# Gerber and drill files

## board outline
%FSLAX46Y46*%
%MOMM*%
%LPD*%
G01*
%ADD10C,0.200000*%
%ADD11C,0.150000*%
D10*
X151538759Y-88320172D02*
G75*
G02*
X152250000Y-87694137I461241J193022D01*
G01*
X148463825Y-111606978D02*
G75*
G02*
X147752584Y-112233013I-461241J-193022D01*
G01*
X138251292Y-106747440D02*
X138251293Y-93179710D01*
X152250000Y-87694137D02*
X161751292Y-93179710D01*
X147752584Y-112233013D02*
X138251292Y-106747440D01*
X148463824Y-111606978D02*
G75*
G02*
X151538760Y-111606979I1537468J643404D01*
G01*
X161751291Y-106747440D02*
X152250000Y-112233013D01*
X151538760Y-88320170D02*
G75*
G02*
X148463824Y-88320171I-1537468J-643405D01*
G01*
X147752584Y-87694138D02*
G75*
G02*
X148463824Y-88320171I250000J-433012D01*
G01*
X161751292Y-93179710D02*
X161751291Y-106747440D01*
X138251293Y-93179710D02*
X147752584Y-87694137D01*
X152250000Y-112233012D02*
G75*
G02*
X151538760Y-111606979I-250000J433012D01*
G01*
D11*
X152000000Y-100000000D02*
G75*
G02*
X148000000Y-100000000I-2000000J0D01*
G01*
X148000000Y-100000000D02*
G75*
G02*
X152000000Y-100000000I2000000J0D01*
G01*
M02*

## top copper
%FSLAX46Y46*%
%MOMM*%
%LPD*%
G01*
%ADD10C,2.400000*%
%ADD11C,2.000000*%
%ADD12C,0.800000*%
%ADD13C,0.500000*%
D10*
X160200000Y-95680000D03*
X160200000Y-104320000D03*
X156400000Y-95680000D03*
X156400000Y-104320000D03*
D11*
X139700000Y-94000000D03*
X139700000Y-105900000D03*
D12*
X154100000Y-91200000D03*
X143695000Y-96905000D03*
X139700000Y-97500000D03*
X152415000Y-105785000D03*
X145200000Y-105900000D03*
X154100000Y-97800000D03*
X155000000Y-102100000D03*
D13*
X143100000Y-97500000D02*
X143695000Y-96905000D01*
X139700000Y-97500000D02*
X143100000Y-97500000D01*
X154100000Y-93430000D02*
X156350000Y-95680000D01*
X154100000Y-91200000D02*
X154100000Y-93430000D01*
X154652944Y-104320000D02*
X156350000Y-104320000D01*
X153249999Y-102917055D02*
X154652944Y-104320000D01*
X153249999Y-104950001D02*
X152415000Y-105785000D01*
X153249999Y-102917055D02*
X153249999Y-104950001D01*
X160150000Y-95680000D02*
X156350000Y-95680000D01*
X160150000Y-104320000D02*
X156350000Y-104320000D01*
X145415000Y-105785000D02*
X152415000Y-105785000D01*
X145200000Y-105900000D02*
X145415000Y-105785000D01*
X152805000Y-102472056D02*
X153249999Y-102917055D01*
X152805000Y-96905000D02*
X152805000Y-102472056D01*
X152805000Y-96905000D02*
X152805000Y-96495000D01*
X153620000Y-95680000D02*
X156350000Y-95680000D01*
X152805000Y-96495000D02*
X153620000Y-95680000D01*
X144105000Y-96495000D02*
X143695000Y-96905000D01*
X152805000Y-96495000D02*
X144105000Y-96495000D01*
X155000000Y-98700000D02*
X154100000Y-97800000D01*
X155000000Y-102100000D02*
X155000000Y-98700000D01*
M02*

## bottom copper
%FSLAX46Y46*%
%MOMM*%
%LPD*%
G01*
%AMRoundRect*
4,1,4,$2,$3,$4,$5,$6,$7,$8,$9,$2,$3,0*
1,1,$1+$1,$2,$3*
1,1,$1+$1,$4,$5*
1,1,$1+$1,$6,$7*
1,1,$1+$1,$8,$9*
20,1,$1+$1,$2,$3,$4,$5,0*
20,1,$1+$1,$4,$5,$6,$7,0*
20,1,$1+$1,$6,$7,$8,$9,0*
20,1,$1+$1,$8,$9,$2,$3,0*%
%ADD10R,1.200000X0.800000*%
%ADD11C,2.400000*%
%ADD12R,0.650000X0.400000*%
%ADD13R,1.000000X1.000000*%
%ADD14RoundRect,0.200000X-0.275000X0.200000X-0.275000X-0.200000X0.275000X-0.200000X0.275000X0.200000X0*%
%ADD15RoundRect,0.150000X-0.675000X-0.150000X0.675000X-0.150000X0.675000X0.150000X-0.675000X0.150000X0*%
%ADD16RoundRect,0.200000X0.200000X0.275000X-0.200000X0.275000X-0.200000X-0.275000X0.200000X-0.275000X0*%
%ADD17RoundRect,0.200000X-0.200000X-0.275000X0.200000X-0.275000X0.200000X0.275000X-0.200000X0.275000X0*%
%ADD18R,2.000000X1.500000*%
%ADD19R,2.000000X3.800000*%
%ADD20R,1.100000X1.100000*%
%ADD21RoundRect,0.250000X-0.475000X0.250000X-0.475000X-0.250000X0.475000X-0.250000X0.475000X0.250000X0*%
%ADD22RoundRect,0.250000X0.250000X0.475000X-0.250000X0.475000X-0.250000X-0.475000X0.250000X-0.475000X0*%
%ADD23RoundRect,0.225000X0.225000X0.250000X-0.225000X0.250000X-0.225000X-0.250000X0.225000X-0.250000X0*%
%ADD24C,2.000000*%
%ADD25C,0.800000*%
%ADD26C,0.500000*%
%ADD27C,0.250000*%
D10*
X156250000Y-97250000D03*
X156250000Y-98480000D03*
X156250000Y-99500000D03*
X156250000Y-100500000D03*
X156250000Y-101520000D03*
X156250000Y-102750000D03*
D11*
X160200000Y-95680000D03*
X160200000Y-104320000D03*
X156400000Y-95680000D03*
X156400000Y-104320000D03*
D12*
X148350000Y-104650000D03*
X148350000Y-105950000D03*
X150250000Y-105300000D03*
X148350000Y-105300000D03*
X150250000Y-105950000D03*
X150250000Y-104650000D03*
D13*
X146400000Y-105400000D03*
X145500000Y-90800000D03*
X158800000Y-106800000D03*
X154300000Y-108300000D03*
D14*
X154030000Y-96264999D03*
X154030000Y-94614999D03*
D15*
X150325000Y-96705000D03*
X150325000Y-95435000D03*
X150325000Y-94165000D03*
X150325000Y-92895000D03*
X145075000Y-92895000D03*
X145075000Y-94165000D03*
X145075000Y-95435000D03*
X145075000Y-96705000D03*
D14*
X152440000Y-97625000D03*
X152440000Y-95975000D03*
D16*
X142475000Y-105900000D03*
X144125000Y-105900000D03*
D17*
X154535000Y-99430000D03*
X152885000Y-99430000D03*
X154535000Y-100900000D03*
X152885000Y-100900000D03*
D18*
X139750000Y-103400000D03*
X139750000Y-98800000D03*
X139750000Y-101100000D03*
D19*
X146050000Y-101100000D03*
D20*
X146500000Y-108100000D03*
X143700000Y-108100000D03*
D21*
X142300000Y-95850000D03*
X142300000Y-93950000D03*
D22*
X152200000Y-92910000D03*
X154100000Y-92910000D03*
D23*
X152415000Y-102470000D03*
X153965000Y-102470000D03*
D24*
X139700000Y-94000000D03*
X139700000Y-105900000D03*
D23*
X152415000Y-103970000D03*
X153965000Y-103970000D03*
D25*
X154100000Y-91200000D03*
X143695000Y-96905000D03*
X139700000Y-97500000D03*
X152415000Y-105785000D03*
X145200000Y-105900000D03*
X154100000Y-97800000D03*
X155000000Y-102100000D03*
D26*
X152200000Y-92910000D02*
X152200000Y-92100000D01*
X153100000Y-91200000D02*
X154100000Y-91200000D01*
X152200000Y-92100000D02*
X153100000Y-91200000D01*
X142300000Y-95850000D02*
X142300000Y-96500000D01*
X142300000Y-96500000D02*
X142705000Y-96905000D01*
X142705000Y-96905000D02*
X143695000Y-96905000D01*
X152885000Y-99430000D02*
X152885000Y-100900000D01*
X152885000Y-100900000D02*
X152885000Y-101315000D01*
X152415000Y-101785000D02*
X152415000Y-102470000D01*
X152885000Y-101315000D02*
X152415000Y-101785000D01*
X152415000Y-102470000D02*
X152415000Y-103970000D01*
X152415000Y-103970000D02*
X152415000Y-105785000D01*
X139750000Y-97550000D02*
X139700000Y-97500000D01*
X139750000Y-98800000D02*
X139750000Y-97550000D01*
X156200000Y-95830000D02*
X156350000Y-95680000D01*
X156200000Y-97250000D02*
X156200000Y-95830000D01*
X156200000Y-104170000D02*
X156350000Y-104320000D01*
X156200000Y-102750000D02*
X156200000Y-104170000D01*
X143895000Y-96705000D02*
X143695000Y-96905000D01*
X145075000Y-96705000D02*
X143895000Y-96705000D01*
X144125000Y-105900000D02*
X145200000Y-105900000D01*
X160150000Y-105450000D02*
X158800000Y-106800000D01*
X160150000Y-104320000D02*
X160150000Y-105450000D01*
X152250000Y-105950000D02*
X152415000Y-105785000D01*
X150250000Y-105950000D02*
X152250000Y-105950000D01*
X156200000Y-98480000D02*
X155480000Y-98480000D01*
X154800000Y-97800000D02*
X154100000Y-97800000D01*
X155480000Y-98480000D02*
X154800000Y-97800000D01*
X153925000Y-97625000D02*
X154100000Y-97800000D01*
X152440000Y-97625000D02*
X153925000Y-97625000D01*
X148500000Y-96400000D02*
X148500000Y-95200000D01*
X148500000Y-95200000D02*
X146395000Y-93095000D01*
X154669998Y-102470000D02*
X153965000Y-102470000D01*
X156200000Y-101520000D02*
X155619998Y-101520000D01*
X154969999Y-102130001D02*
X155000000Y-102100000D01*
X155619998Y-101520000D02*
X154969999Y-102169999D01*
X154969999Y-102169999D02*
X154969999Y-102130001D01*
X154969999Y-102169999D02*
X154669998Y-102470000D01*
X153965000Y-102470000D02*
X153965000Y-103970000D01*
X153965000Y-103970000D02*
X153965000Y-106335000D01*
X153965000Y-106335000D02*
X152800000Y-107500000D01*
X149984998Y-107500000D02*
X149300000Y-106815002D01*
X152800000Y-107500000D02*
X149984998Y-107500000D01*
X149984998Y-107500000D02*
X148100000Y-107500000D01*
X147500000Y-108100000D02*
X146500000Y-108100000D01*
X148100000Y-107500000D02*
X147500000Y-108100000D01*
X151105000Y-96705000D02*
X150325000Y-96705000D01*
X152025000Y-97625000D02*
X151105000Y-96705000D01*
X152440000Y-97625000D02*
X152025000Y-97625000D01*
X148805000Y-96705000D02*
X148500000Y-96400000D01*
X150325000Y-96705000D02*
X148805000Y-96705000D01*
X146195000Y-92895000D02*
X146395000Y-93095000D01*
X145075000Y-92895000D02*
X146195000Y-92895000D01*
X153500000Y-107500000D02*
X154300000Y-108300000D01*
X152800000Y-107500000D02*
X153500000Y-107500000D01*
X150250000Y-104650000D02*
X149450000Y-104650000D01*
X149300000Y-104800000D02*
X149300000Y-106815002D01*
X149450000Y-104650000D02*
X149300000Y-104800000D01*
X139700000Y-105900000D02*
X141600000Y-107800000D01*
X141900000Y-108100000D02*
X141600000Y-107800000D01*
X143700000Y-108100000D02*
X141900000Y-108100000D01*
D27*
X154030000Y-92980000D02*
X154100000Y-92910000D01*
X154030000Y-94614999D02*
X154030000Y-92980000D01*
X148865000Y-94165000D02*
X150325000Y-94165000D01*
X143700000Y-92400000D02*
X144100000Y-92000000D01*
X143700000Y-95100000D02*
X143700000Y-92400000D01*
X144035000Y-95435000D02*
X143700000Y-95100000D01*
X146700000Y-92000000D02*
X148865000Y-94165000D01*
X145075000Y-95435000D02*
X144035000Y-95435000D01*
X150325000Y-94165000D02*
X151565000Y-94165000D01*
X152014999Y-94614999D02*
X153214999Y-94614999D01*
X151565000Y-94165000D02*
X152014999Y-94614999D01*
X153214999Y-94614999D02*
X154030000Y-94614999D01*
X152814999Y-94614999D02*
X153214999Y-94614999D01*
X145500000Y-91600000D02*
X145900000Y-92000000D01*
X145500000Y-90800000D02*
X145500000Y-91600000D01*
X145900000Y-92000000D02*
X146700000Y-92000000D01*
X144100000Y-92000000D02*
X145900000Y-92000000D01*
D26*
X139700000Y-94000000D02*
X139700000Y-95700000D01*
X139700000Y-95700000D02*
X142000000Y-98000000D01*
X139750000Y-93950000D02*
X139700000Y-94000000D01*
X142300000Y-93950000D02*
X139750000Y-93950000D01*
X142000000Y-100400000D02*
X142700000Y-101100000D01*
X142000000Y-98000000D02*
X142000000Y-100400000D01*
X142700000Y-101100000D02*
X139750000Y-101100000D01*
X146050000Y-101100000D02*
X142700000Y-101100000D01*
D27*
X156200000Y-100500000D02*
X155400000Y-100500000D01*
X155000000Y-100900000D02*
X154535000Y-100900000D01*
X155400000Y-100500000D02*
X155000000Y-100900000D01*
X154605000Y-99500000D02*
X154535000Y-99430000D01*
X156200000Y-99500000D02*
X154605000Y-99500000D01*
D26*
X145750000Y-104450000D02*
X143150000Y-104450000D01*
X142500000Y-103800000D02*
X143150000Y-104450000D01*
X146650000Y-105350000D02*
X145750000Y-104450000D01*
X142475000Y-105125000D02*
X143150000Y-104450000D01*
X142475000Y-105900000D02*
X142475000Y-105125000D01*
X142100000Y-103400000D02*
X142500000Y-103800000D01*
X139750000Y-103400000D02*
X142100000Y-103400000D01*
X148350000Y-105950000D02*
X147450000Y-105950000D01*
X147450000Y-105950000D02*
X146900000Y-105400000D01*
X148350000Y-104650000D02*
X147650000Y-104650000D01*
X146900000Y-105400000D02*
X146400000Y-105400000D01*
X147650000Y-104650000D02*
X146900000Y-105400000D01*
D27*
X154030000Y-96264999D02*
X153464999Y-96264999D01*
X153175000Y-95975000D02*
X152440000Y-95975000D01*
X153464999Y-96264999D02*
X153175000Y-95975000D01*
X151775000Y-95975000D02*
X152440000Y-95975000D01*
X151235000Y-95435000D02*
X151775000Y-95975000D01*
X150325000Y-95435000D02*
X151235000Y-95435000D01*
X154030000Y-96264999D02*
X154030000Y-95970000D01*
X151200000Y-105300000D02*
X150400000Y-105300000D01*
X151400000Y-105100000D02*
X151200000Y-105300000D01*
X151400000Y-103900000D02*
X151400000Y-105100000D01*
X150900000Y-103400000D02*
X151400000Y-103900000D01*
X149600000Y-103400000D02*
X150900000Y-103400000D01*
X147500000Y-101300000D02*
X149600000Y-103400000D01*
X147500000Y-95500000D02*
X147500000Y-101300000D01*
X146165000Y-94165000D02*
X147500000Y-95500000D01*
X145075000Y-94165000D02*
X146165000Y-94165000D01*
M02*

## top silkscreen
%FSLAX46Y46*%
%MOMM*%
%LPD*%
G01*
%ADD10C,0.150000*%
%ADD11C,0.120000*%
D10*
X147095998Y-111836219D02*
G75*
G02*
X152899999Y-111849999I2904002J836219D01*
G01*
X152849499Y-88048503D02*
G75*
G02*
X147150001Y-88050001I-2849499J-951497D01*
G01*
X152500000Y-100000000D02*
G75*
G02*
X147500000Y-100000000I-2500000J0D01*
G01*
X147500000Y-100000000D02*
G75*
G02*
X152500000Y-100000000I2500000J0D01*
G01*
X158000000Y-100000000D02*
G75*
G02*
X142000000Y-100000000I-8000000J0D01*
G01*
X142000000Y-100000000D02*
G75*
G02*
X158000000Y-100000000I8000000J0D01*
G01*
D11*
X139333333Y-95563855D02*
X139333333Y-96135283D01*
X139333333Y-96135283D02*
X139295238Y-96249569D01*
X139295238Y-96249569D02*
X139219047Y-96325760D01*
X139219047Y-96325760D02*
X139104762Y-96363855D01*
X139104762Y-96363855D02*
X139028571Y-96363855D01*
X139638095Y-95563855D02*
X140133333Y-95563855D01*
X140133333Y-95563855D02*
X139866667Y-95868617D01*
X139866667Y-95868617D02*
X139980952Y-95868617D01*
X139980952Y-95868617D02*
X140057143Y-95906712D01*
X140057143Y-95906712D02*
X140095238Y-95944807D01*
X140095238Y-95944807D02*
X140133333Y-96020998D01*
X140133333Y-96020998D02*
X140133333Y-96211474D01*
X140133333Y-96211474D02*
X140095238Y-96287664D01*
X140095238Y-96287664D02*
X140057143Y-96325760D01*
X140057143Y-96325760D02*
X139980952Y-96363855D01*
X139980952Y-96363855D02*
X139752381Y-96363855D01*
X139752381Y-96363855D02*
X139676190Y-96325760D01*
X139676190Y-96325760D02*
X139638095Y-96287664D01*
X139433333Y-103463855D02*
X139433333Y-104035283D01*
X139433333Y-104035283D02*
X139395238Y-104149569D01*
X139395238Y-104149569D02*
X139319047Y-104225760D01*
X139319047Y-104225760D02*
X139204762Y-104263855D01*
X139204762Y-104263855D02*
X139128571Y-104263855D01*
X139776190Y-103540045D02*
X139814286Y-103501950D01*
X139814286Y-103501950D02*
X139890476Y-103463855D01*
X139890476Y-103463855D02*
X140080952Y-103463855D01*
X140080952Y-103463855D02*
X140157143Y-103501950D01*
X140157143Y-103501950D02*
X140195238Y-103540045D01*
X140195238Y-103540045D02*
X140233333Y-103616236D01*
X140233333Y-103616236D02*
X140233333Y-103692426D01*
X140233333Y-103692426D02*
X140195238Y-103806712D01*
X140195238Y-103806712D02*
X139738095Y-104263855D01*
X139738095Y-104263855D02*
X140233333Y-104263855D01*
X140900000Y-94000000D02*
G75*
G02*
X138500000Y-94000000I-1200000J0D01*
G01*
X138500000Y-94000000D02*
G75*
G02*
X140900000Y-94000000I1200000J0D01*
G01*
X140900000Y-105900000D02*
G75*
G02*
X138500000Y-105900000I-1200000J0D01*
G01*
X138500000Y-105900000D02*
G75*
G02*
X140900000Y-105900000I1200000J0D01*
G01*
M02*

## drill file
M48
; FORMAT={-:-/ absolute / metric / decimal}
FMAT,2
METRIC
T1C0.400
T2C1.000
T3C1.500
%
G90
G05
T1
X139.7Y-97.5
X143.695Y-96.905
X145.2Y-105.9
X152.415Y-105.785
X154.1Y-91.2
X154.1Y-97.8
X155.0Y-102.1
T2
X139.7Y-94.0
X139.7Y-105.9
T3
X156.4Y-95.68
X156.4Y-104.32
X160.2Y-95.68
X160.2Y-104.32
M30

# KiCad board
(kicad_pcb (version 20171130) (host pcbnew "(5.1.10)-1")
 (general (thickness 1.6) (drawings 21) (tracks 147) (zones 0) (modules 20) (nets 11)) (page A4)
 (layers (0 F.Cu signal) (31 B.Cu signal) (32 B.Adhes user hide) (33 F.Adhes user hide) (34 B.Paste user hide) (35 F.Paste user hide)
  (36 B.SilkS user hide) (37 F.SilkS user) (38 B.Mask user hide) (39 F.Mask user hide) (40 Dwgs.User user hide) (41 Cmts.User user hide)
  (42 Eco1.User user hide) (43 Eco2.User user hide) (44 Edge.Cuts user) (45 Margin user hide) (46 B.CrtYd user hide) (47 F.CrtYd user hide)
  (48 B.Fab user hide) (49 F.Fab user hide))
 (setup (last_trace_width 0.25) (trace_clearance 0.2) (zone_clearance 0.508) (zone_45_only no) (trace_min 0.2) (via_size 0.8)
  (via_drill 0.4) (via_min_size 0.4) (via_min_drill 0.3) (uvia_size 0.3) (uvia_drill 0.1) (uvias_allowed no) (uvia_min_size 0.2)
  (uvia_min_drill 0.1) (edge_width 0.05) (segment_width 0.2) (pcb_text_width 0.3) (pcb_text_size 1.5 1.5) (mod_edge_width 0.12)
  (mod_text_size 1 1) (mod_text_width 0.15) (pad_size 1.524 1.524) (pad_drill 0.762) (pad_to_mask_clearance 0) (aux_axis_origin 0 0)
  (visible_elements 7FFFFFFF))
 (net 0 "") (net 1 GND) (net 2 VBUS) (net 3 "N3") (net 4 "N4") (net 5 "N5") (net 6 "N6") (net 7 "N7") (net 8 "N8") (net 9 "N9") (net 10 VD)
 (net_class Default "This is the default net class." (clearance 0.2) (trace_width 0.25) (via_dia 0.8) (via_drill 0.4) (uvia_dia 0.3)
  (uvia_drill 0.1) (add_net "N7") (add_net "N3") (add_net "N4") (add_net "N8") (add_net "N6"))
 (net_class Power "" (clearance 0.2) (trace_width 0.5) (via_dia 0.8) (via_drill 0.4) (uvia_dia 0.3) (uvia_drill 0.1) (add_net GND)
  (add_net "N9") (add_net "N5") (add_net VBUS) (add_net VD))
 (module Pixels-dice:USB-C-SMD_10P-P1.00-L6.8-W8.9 (layer B.Cu) (at 158.3 100 180)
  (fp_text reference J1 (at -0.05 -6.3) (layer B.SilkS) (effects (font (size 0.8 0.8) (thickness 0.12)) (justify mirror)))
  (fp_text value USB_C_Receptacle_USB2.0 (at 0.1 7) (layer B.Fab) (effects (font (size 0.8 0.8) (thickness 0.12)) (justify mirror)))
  (pad B12 smd rect (at 2.05 2.75 270) (size 0.8 1.2) (layers B.Cu B.Paste B.Mask) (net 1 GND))
  (pad B9 smd rect (at 2.05 1.52 270) (size 0.8 1.2) (layers B.Cu B.Paste B.Mask) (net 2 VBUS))
  (pad A5 smd rect (at 2.05 0.5 270) (size 0.8 1.2) (layers B.Cu B.Paste B.Mask) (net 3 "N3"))
  (pad B5 smd rect (at 2.05 -0.5 270) (size 0.8 1.2) (layers B.Cu B.Paste B.Mask) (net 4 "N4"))
  (pad A9 smd rect (at 2.05 -1.52 270) (size 0.8 1.2) (layers B.Cu B.Paste B.Mask) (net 2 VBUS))
  (pad A12 smd rect (at 2.05 -2.75 270) (size 0.8 1.2) (layers B.Cu B.Paste B.Mask) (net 1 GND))
  (pad S1 thru_hole circle (at -1.9 4.32 270) (size 2.4 2.4) (drill 1.5) (layers *.Cu *.Mask) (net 1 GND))
  (pad S1 thru_hole circle (at -1.9 -4.32 270) (size 2.4 2.4) (drill 1.5) (layers *.Cu *.Mask) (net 1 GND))
  (pad S1 thru_hole circle (at 1.9 4.32 270) (size 2.4 2.4) (drill 1.5) (layers *.Cu *.Mask) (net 1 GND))
  (pad S1 thru_hole circle (at 1.9 -4.32 270) (size 2.4 2.4) (drill 1.5) (layers *.Cu *.Mask) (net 1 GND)))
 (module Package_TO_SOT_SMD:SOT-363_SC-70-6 (layer B.Cu) (at 149.3 105.3 180)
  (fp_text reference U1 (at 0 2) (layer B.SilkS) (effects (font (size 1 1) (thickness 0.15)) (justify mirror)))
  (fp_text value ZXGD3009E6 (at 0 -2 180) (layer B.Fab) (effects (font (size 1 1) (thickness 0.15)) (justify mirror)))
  (pad 6 smd rect (at 0.95 0.65 180) (size 0.65 0.4) (layers B.Cu B.Paste B.Mask) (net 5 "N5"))
  (pad 4 smd rect (at 0.95 -0.65 180) (size 0.65 0.4) (layers B.Cu B.Paste B.Mask) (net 5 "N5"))
  (pad 2 smd rect (at -0.95 0 180) (size 0.65 0.4) (layers B.Cu B.Paste B.Mask) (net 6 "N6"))
  (pad 5 smd rect (at 0.95 0 180) (size 0.65 0.4) (layers B.Cu B.Paste B.Mask))
  (pad 3 smd rect (at -0.95 -0.65 180) (size 0.65 0.4) (layers B.Cu B.Paste B.Mask) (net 1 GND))
  (pad 1 smd rect (at -0.95 0.65 180) (size 0.65 0.4) (layers B.Cu B.Paste B.Mask) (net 2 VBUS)))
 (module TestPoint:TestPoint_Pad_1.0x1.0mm (layer B.Cu) (at 146.4 105.4)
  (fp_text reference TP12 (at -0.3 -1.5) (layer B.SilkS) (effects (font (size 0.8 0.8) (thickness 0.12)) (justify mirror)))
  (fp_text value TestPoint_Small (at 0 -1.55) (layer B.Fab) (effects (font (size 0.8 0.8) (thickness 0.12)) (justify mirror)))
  (pad 1 smd rect (at 0 0) (size 1 1) (layers B.Cu B.Mask) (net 5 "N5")))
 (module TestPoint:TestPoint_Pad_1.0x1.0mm (layer B.Cu) (at 145.5 90.8)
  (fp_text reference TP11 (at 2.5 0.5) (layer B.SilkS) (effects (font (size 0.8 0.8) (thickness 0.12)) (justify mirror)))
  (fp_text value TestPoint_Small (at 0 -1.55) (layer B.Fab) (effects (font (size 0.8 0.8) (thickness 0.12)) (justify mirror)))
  (pad 1 smd rect (at 0 0) (size 1 1) (layers B.Cu B.Mask) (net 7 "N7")))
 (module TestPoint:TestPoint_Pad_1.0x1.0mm (layer B.Cu) (at 158.8 106.8)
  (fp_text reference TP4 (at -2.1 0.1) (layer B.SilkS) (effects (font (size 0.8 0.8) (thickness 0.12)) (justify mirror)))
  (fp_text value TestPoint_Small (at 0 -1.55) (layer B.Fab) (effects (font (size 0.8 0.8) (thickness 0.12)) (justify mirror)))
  (pad 1 smd rect (at 0 0) (size 1 1) (layers B.Cu B.Mask) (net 1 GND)))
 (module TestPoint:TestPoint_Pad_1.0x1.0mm (layer B.Cu) (at 154.3 108.3)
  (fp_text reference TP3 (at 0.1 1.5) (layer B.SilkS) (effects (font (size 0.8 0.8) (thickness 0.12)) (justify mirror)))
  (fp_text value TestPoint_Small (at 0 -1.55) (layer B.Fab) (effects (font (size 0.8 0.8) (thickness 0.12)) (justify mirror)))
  (pad 1 smd rect (at 0 0) (size 1 1) (layers B.Cu B.Mask) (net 2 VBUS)))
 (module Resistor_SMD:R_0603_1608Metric (layer B.Cu) (at 154.03 95.439999 270)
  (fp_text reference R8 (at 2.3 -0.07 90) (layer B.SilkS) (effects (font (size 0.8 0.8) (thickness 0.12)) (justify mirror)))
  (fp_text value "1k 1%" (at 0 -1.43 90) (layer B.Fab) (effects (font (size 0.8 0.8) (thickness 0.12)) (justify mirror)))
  (pad 2 smd roundrect (at 0.825 0 270) (size 0.8 0.95) (layers B.Cu B.Paste B.Mask) (roundrect_rratio 0.25) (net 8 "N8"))
  (pad 1 smd roundrect (at -0.825 0 270) (size 0.8 0.95) (layers B.Cu B.Paste B.Mask) (roundrect_rratio 0.25) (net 7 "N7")))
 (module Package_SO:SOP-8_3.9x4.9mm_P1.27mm (layer B.Cu) (at 147.7 94.8)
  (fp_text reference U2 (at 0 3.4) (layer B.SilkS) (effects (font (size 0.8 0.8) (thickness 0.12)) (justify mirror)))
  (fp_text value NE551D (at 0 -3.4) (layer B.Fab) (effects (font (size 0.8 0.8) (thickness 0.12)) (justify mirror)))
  (pad 8 smd roundrect (at 2.625 1.905) (size 1.65 0.6) (layers B.Cu B.Paste B.Mask) (roundrect_rratio 0.25) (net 2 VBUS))
  (pad 7 smd roundrect (at 2.625 0.635) (size 1.65 0.6) (layers B.Cu B.Paste B.Mask) (roundrect_rratio 0.25) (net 8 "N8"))
  (pad 6 smd roundrect (at 2.625 -0.635) (size 1.65 0.6) (layers B.Cu B.Paste B.Mask) (roundrect_rratio 0.25) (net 7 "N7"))
  (pad 5 smd roundrect (at 2.625 -1.905) (size 1.65 0.6) (layers B.Cu B.Paste B.Mask) (roundrect_rratio 0.25))
  (pad 4 smd roundrect (at -2.625 -1.905) (size 1.65 0.6) (layers B.Cu B.Paste B.Mask) (roundrect_rratio 0.25) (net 2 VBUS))
  (pad 3 smd roundrect (at -2.625 -0.635) (size 1.65 0.6) (layers B.Cu B.Paste B.Mask) (roundrect_rratio 0.25) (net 6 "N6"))
  (pad 2 smd roundrect (at -2.625 0.635) (size 1.65 0.6) (layers B.Cu B.Paste B.Mask) (roundrect_rratio 0.25) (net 7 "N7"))
  (pad 1 smd roundrect (at -2.625 1.905) (size 1.65 0.6) (layers B.Cu B.Paste B.Mask) (roundrect_rratio 0.25) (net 1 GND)))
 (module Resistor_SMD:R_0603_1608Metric (layer B.Cu) (at 152.44 96.8 270)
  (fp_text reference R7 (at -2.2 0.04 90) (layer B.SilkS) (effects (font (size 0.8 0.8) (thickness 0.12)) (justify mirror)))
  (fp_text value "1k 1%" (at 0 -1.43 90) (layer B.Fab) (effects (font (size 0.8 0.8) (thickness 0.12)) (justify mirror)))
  (pad 2 smd roundrect (at 0.825 0 270) (size 0.8 0.95) (layers B.Cu B.Paste B.Mask) (roundrect_rratio 0.25) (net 2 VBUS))
  (pad 1 smd roundrect (at -0.825 0 270) (size 0.8 0.95) (layers B.Cu B.Paste B.Mask) (roundrect_rratio 0.25) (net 8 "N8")))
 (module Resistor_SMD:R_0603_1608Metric (layer B.Cu) (at 143.3 105.9 180)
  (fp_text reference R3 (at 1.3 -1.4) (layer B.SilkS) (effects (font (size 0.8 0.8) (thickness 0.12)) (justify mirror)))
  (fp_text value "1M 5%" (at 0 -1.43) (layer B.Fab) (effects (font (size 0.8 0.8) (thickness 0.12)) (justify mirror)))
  (pad 2 smd roundrect (at 0.825 0 180) (size 0.8 0.95) (layers B.Cu B.Paste B.Mask) (roundrect_rratio 0.25) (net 5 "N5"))
  (pad 1 smd roundrect (at -0.825 0 180) (size 0.8 0.95) (layers B.Cu B.Paste B.Mask) (roundrect_rratio 0.25) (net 1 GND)))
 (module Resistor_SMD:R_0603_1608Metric (layer B.Cu) (at 153.71 99.43)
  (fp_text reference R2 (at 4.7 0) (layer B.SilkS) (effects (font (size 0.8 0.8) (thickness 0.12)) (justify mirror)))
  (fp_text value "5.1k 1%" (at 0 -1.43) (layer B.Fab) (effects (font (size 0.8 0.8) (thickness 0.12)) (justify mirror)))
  (pad 2 smd roundrect (at 0.825 0) (size 0.8 0.95) (layers B.Cu B.Paste B.Mask) (roundrect_rratio 0.25) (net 3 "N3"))
  (pad 1 smd roundrect (at -0.825 0) (size 0.8 0.95) (layers B.Cu B.Paste B.Mask) (roundrect_rratio 0.25) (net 1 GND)))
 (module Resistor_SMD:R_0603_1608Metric (layer B.Cu) (at 153.71 100.9)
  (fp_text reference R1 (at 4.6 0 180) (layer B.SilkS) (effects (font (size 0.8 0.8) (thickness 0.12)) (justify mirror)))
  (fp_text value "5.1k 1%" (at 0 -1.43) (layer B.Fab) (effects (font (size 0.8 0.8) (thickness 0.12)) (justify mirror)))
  (pad 2 smd roundrect (at 0.825 0) (size 0.8 0.95) (layers B.Cu B.Paste B.Mask) (roundrect_rratio 0.25) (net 4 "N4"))
  (pad 1 smd roundrect (at -0.825 0) (size 0.8 0.95) (layers B.Cu B.Paste B.Mask) (roundrect_rratio 0.25) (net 1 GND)))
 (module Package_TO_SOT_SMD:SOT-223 (layer B.Cu) (at 142.9 101.1)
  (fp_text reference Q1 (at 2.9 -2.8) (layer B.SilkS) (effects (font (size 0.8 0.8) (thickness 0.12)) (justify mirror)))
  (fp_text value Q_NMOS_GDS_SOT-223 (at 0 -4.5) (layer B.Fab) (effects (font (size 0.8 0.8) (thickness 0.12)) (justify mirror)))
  (pad 1 smd rect (at -3.15 2.3) (size 2 1.5) (layers B.Cu B.Paste B.Mask) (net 5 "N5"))
  (pad 3 smd rect (at -3.15 -2.3) (size 2 1.5) (layers B.Cu B.Paste B.Mask) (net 1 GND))
  (pad 2 smd rect (at -3.15 0) (size 2 1.5) (layers B.Cu B.Paste B.Mask) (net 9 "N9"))
  (pad 4 smd rect (at 3.15 0) (size 2 3.8) (layers B.Cu B.Paste B.Mask) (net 9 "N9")))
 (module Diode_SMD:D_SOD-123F (layer B.Cu) (at 145.1 108.1)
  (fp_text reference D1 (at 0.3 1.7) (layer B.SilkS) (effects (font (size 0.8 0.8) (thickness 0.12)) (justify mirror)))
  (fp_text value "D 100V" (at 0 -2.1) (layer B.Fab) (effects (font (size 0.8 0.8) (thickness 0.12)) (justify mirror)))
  (pad 2 smd rect (at 1.4 0) (size 1.1 1.1) (layers B.Cu B.Paste B.Mask) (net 2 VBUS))
  (pad 1 smd rect (at -1.4 0) (size 1.1 1.1) (layers B.Cu B.Paste B.Mask) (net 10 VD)))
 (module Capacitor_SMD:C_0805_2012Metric (layer B.Cu) (at 142.3 94.9 270)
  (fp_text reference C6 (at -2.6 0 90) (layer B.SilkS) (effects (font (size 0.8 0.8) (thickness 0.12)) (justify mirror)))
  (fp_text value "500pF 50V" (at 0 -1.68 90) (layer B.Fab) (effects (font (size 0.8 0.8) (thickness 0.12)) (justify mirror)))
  (pad 2 smd roundrect (at 0.95 0 270) (size 1 1.45) (layers B.Cu B.Paste B.Mask) (roundrect_rratio 0.25) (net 1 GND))
  (pad 1 smd roundrect (at -0.95 0 270) (size 1 1.45) (layers B.Cu B.Paste B.Mask) (roundrect_rratio 0.25) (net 9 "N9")))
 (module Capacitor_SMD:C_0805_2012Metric (layer B.Cu) (at 153.15 92.91 180)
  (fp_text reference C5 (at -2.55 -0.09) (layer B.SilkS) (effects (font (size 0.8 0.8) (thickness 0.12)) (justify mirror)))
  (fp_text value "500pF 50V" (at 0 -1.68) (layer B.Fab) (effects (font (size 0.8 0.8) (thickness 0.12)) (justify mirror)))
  (pad 2 smd roundrect (at 0.95 0 180) (size 1 1.45) (layers B.Cu B.Paste B.Mask) (roundrect_rratio 0.25) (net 1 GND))
  (pad 1 smd roundrect (at -0.95 0 180) (size 1 1.45) (layers B.Cu B.Paste B.Mask) (roundrect_rratio 0.25) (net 7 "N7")))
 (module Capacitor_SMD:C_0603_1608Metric (layer B.Cu) (at 153.19 102.47 180)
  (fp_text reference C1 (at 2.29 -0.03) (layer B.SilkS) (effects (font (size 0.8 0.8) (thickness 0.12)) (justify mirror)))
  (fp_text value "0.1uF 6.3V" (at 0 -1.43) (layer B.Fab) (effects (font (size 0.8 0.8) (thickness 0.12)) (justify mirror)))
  (pad 2 smd roundrect (at 0.775 0 180) (size 0.9 0.95) (layers B.Cu B.Paste B.Mask) (roundrect_rratio 0.25) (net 1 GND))
  (pad 1 smd roundrect (at -0.775 0 180) (size 0.9 0.95) (layers B.Cu B.Paste B.Mask) (roundrect_rratio 0.25) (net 2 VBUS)))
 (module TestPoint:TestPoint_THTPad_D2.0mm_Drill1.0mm (layer F.Cu) (at 139.7 94)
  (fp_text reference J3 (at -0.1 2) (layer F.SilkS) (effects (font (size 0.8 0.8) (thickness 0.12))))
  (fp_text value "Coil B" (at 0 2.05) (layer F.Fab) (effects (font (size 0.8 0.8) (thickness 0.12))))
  (fp_circle (center 0 0) (end 0 1.2) (layer F.SilkS) (width 0.12))
  (pad 1 thru_hole circle (at 0 0) (size 2 2) (drill 1) (layers *.Cu *.Mask) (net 9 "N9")))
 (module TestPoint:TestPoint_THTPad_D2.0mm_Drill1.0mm (layer F.Cu) (at 139.7 105.9)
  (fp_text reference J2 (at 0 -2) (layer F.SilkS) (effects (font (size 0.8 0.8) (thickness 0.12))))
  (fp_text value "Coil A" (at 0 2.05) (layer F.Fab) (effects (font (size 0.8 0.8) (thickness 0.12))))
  (fp_circle (center 0 0) (end 0 1.2) (layer F.SilkS) (width 0.12))
  (pad 1 thru_hole circle (at 0 0) (size 2 2) (drill 1) (layers *.Cu *.Mask) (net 10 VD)))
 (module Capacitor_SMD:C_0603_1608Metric (layer B.Cu) (at 153.19 103.97 180)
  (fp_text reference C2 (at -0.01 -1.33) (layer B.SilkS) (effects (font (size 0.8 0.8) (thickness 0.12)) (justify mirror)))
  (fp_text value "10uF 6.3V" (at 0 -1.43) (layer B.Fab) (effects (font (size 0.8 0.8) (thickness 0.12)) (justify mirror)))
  (pad 2 smd roundrect (at 0.775 0 180) (size 0.9 0.95) (layers B.Cu B.Paste B.Mask) (roundrect_rratio 0.25) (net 1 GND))
  (pad 1 smd roundrect (at -0.775 0 180) (size 0.9 0.95) (layers B.Cu B.Paste B.Mask) (roundrect_rratio 0.25) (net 2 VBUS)))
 (gr_arc (start 150 111) (end 152.899999 111.849999) (angle -212.4) (layer F.SilkS) (width 0.15))
 (gr_arc (start 150 89) (end 147.150001 88.050001) (angle -216.9) (layer F.SilkS) (width 0.15))
 (gr_arc (start 152 88.12715) (end 152.25 87.694137) (angle -142.7084941) (layer Edge.Cuts) (width 0.2))
 (gr_arc (start 148.002584 111.8) (end 147.752584 112.233013) (angle -142.7084941) (layer Edge.Cuts) (width 0.2))
 (gr_line (start 138.251292 106.74744) (end 138.251293 93.17971) (layer Edge.Cuts) (width 0.2))
 (gr_line (start 152.25 87.694137) (end 161.751292 93.17971) (layer Edge.Cuts) (width 0.2))
 (gr_line (start 147.752584 112.233013) (end 138.251292 106.74744) (layer Edge.Cuts) (width 0.2))
 (gr_arc (start 150.001292 110.963574) (end 151.53876 111.606979) (angle -225.4169678) (layer Edge.Cuts) (width 0.2))
 (gr_line (start 161.751291 106.74744) (end 152.25 112.233013) (layer Edge.Cuts) (width 0.2))
 (gr_arc (start 150.001292 88.963575) (end 148.463824 88.320171) (angle -225.4169678) (layer Edge.Cuts) (width 0.2))
 (gr_arc (start 148.002584 88.12715) (end 148.463824 88.320171) (angle -142.7084738) (layer Edge.Cuts) (width 0.2))
 (gr_line (start 161.751292 93.17971) (end 161.751291 106.74744) (layer Edge.Cuts) (width 0.2))
 (gr_line (start 138.251293 93.17971) (end 147.752584 87.694137) (layer Edge.Cuts) (width 0.2))
 (gr_arc (start 152 111.8) (end 151.53876 111.606979) (angle -142.7084738) (layer Edge.Cuts) (width 0.2))
 (gr_circle (center 150 100) (end 152 100) (layer Edge.Cuts) (width 0.15))
 (gr_circle (center 150 100) (end 152.5 100) (layer F.SilkS) (width 0.15))
 (gr_circle (center 150 100) (end 158 100) (layer F.SilkS) (width 0.15))
 (segment (start 152.2 92.91) (end 152.2 92.1) (width 0.5) (layer B.Cu) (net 1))
 (via (at 154.1 91.2) (size 0.8) (drill 0.4) (layers F.Cu B.Cu) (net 1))
 (segment (start 153.1 91.2) (end 154.1 91.2) (width 0.5) (layer B.Cu) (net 1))
 (segment (start 152.2 92.1) (end 153.1 91.2) (width 0.5) (layer B.Cu) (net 1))
 (segment (start 142.3 95.85) (end 142.3 96.5) (width 0.5) (layer B.Cu) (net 1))
 (segment (start 142.3 96.5) (end 142.705 96.905) (width 0.5) (layer B.Cu) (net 1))
 (via (at 143.695 96.905) (size 0.8) (drill 0.4) (layers F.Cu B.Cu) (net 1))
 (segment (start 142.705 96.905) (end 143.695 96.905) (width 0.5) (layer B.Cu) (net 1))
 (via (at 139.7 97.5) (size 0.8) (drill 0.4) (layers F.Cu B.Cu) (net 1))
 (segment (start 152.885 99.43) (end 152.885 100.9) (width 0.5) (layer B.Cu) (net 1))
 (segment (start 152.885 100.9) (end 152.885 101.315) (width 0.5) (layer B.Cu) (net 1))
 (segment (start 152.415 101.785) (end 152.415 102.47) (width 0.5) (layer B.Cu) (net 1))
 (segment (start 152.885 101.315) (end 152.415 101.785) (width 0.5) (layer B.Cu) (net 1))
 (segment (start 152.415 102.47) (end 152.415 103.97) (width 0.5) (layer B.Cu) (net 1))
 (segment (start 152.415 103.97) (end 152.415 105.785) (width 0.5) (layer B.Cu) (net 1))
 (via (at 152.415 105.785) (size 0.8) (drill 0.4) (layers F.Cu B.Cu) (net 1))
 (segment (start 139.75 97.55) (end 139.7 97.5) (width 0.5) (layer B.Cu) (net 1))
 (segment (start 139.75 98.8) (end 139.75 97.55) (width 0.5) (layer B.Cu) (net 1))
 (segment (start 143.1 97.5) (end 143.695 96.905) (width 0.5) (layer F.Cu) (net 1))
 (segment (start 139.7 97.5) (end 143.1 97.5) (width 0.5) (layer F.Cu) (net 1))
 (segment (start 154.1 93.43) (end 156.35 95.68) (width 0.5) (layer F.Cu) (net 1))
 (segment (start 154.1 91.2) (end 154.1 93.43) (width 0.5) (layer F.Cu) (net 1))
 (segment (start 156.2 95.83) (end 156.35 95.68) (width 0.5) (layer B.Cu) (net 1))
 (segment (start 156.2 97.25) (end 156.2 95.83) (width 0.5) (layer B.Cu) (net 1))
 (segment (start 156.2 104.17) (end 156.35 104.32) (width 0.5) (layer B.Cu) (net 1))
 (segment (start 156.2 102.75) (end 156.2 104.17) (width 0.5) (layer B.Cu) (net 1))
 (segment (start 154.652944 104.32) (end 156.35 104.32) (width 0.5) (layer F.Cu) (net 1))
 (segment (start 153.249999 102.917055) (end 154.652944 104.32) (width 0.5) (layer F.Cu) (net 1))
 (segment (start 153.249999 104.950001) (end 152.415 105.785) (width 0.5) (layer F.Cu) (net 1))
 (segment (start 153.249999 102.917055) (end 153.249999 104.950001) (width 0.5) (layer F.Cu) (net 1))
 (segment (start 160.15 95.68) (end 156.35 95.68) (width 0.5) (layer F.Cu) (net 1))
 (segment (start 160.15 104.32) (end 156.35 104.32) (width 0.5) (layer F.Cu) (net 1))
 (segment (start 143.895 96.705) (end 143.695 96.905) (width 0.5) (layer B.Cu) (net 1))
 (segment (start 145.075 96.705) (end 143.895 96.705) (width 0.5) (layer B.Cu) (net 1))
 (segment (start 145.415 105.785) (end 152.415 105.785) (width 0.5) (layer F.Cu) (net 1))
 (segment (start 145.2 105.9) (end 145.415 105.785) (width 0.5) (layer F.Cu) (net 1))
 (segment (start 144.125 105.9) (end 145.2 105.9) (width 0.5) (layer B.Cu) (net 1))
 (via (at 145.2 105.9) (size 0.8) (drill 0.4) (layers F.Cu B.Cu) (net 1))
 (segment (start 160.15 105.45) (end 158.8 106.8) (width 0.5) (layer B.Cu) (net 1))
 (segment (start 160.15 104.32) (end 160.15 105.45) (width 0.5) (layer B.Cu) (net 1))
 (segment (start 152.805 102.472056) (end 153.249999 102.917055) (width 0.5) (layer F.Cu) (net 1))
 (segment (start 152.805 96.905) (end 152.805 102.472056) (width 0.5) (layer F.Cu) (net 1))
 (segment (start 152.805 96.905) (end 152.805 96.495) (width 0.5) (layer F.Cu) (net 1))
 (segment (start 153.62 95.68) (end 156.35 95.68) (width 0.5) (layer F.Cu) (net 1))
 (segment (start 152.805 96.495) (end 153.62 95.68) (width 0.5) (layer F.Cu) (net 1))
 (segment (start 144.105 96.495) (end 143.695 96.905) (width 0.5) (layer F.Cu) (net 1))
 (segment (start 152.805 96.495) (end 144.105 96.495) (width 0.5) (layer F.Cu) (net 1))
 (segment (start 152.25 105.95) (end 152.415 105.785) (width 0.5) (layer B.Cu) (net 1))
 (segment (start 150.25 105.95) (end 152.25 105.95) (width 0.5) (layer B.Cu) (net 1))
 (segment (start 156.2 98.48) (end 155.48 98.48) (width 0.5) (layer B.Cu) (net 2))
 (segment (start 154.8 97.8) (end 154.1 97.8) (width 0.5) (layer B.Cu) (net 2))
 (via (at 154.1 97.8) (size 0.8) (drill 0.4) (layers F.Cu B.Cu) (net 2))
 (segment (start 155.48 98.48) (end 154.8 97.8) (width 0.5) (layer B.Cu) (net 2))
 (segment (start 153.925 97.625) (end 154.1 97.8) (width 0.5) (layer B.Cu) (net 2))
 (segment (start 152.44 97.625) (end 153.925 97.625) (width 0.5) (layer B.Cu) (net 2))
 (segment (start 148.5 96.4) (end 148.5 95.2) (width 0.5) (layer B.Cu) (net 2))
 (segment (start 148.5 95.2) (end 146.395 93.095) (width 0.5) (layer B.Cu) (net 2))
 (segment (start 154.669998 102.47) (end 153.965 102.47) (width 0.5) (layer B.Cu) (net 2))
 (segment (start 156.2 101.52) (end 155.619998 101.52) (width 0.5) (layer B.Cu) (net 2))
 (via (at 155 102.1) (size 0.8) (drill 0.4) (layers F.Cu B.Cu) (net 2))
 (segment (start 154.969999 102.130001) (end 155 102.1) (width 0.5) (layer B.Cu) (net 2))
 (segment (start 155.619998 101.52) (end 154.969999 102.169999) (width 0.5) (layer B.Cu) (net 2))
 (segment (start 154.969999 102.169999) (end 154.969999 102.130001) (width 0.5) (layer B.Cu) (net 2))
 (segment (start 154.969999 102.169999) (end 154.669998 102.47) (width 0.5) (layer B.Cu) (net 2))
 (segment (start 153.965 102.47) (end 153.965 103.97) (width 0.5) (layer B.Cu) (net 2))
 (segment (start 153.965 103.97) (end 153.965 106.335) (width 0.5) (layer B.Cu) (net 2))
 (segment (start 153.965 106.335) (end 152.8 107.5) (width 0.5) (layer B.Cu) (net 2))
 (segment (start 149.984998 107.5) (end 149.3 106.815002) (width 0.5) (layer B.Cu) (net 2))
 (segment (start 152.8 107.5) (end 149.984998 107.5) (width 0.5) (layer B.Cu) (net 2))
 (segment (start 149.984998 107.5) (end 148.1 107.5) (width 0.5) (layer B.Cu) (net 2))
 (segment (start 147.5 108.1) (end 146.5 108.1) (width 0.5) (layer B.Cu) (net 2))
 (segment (start 148.1 107.5) (end 147.5 108.1) (width 0.5) (layer B.Cu) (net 2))
 (segment (start 155 98.7) (end 154.1 97.8) (width 0.5) (layer F.Cu) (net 2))
 (segment (start 155 102.1) (end 155 98.7) (width 0.5) (layer F.Cu) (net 2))
 (segment (start 151.105 96.705) (end 150.325 96.705) (width 0.5) (layer B.Cu) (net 2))
 (segment (start 152.025 97.625) (end 151.105 96.705) (width 0.5) (layer B.Cu) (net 2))
 (segment (start 152.44 97.625) (end 152.025 97.625) (width 0.5) (layer B.Cu) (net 2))
 (segment (start 148.805 96.705) (end 148.5 96.4) (width 0.5) (layer B.Cu) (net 2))
 (segment (start 150.325 96.705) (end 148.805 96.705) (width 0.5) (layer B.Cu) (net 2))
 (segment (start 146.195 92.895) (end 146.395 93.095) (width 0.5) (layer B.Cu) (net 2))
 (segment (start 145.075 92.895) (end 146.195 92.895) (width 0.5) (layer B.Cu) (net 2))
 (segment (start 153.5 107.5) (end 154.3 108.3) (width 0.5) (layer B.Cu) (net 2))
 (segment (start 152.8 107.5) (end 153.5 107.5) (width 0.5) (layer B.Cu) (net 2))
 (segment (start 150.25 104.65) (end 149.45 104.65) (width 0.5) (layer B.Cu) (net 2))
 (segment (start 149.3 104.8) (end 149.3 106.815002) (width 0.5) (layer B.Cu) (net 2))
 (segment (start 149.45 104.65) (end 149.3 104.8) (width 0.5) (layer B.Cu) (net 2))
 (segment (start 139.7 105.9) (end 141.6 107.8) (width 0.5) (layer B.Cu) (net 10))
 (segment (start 141.9 108.1) (end 141.6 107.8) (width 0.5) (layer B.Cu) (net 10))
 (segment (start 143.7 108.1) (end 141.9 108.1) (width 0.5) (layer B.Cu) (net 10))
 (segment (start 154.03 92.98) (end 154.1 92.91) (width 0.25) (layer B.Cu) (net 7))
 (segment (start 154.03 94.614999) (end 154.03 92.98) (width 0.25) (layer B.Cu) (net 7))
 (segment (start 148.865 94.165) (end 150.325 94.165) (width 0.25) (layer B.Cu) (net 7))
 (segment (start 143.7 92.4) (end 144.1 92) (width 0.25) (layer B.Cu) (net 7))
 (segment (start 143.7 95.1) (end 143.7 92.4) (width 0.25) (layer B.Cu) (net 7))
 (segment (start 144.035 95.435) (end 143.7 95.1) (width 0.25) (layer B.Cu) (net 7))
 (segment (start 146.7 92) (end 148.865 94.165) (width 0.25) (layer B.Cu) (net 7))
 (segment (start 145.075 95.435) (end 144.035 95.435) (width 0.25) (layer B.Cu) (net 7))
 (segment (start 150.325 94.165) (end 151.565 94.165) (width 0.25) (layer B.Cu) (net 7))
 (segment (start 152.014999 94.614999) (end 153.214999 94.614999) (width 0.25) (layer B.Cu) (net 7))
 (segment (start 151.565 94.165) (end 152.014999 94.614999) (width 0.25) (layer B.Cu) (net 7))
 (segment (start 153.214999 94.614999) (end 154.03 94.614999) (width 0.25) (layer B.Cu) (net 7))
 (segment (start 152.814999 94.614999) (end 153.214999 94.614999) (width 0.25) (layer B.Cu) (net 7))
 (segment (start 145.5 91.6) (end 145.9 92) (width 0.25) (layer B.Cu) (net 7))
 (segment (start 145.5 90.8) (end 145.5 91.6) (width 0.25) (layer B.Cu) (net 7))
 (segment (start 145.9 92) (end 146.7 92) (width 0.25) (layer B.Cu) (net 7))
 (segment (start 144.1 92) (end 145.9 92) (width 0.25) (layer B.Cu) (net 7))
 (segment (start 139.7 94) (end 139.7 95.7) (width 0.5) (layer B.Cu) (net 9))
 (segment (start 139.7 95.7) (end 142 98) (width 0.5) (layer B.Cu) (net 9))
 (segment (start 139.75 93.95) (end 139.7 94) (width 0.5) (layer B.Cu) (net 9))
 (segment (start 142.3 93.95) (end 139.75 93.95) (width 0.5) (layer B.Cu) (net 9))
 (segment (start 142 100.4) (end 142.7 101.1) (width 0.5) (layer B.Cu) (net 9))
 (segment (start 142 98) (end 142 100.4) (width 0.5) (layer B.Cu) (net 9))
 (segment (start 142.7 101.1) (end 139.75 101.1) (width 0.5) (layer B.Cu) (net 9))
 (segment (start 146.05 101.1) (end 142.7 101.1) (width 0.5) (layer B.Cu) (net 9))
 (segment (start 156.2 100.5) (end 155.4 100.5) (width 0.25) (layer B.Cu) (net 4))
 (segment (start 155 100.9) (end 154.535 100.9) (width 0.25) (layer B.Cu) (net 4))
 (segment (start 155.4 100.5) (end 155 100.9) (width 0.25) (layer B.Cu) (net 4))
 (segment (start 154.605 99.5) (end 154.535 99.43) (width 0.25) (layer B.Cu) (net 3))
 (segment (start 156.2 99.5) (end 154.605 99.5) (width 0.25) (layer B.Cu) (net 3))
 (segment (start 145.75 104.45) (end 143.15 104.45) (width 0.5) (layer B.Cu) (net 5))
 (segment (start 142.5 103.8) (end 143.15 104.45) (width 0.5) (layer B.Cu) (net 5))
 (segment (start 146.65 105.35) (end 145.75 104.45) (width 0.5) (layer B.Cu) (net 5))
 (segment (start 142.475 105.125) (end 143.15 104.45) (width 0.5) (layer B.Cu) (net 5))
 (segment (start 142.475 105.9) (end 142.475 105.125) (width 0.5) (layer B.Cu) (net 5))
 (segment (start 142.1 103.4) (end 142.5 103.8) (width 0.5) (layer B.Cu) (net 5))
 (segment (start 139.75 103.4) (end 142.1 103.4) (width 0.5) (layer B.Cu) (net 5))
 (segment (start 148.35 105.95) (end 147.45 105.95) (width 0.5) (layer B.Cu) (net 5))
 (segment (start 147.45 105.95) (end 146.9 105.4) (width 0.5) (layer B.Cu) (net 5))
 (segment (start 148.35 104.65) (end 147.65 104.65) (width 0.5) (layer B.Cu) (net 5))
 (segment (start 146.9 105.4) (end 146.4 105.4) (width 0.5) (layer B.Cu) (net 5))
 (segment (start 147.65 104.65) (end 146.9 105.4) (width 0.5) (layer B.Cu) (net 5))
 (segment (start 154.03 96.264999) (end 153.464999 96.264999) (width 0.25) (layer B.Cu) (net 8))
 (segment (start 153.175 95.975) (end 152.44 95.975) (width 0.25) (layer B.Cu) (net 8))
 (segment (start 153.464999 96.264999) (end 153.175 95.975) (width 0.25) (layer B.Cu) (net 8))
 (segment (start 151.775 95.975) (end 152.44 95.975) (width 0.25) (layer B.Cu) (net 8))
 (segment (start 151.235 95.435) (end 151.775 95.975) (width 0.25) (layer B.Cu) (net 8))
 (segment (start 150.325 95.435) (end 151.235 95.435) (width 0.25) (layer B.Cu) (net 8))
 (segment (start 154.03 96.264999) (end 154.03 95.97) (width 0.25) (layer B.Cu) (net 8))
 (segment (start 151.2 105.3) (end 150.4 105.3) (width 0.25) (layer B.Cu) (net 6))
 (segment (start 151.4 105.1) (end 151.2 105.3) (width 0.25) (layer B.Cu) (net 6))
 (segment (start 151.4 103.9) (end 151.4 105.1) (width 0.25) (layer B.Cu) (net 6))
 (segment (start 150.9 103.4) (end 151.4 103.9) (width 0.25) (layer B.Cu) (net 6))
 (segment (start 149.6 103.4) (end 150.9 103.4) (width 0.25) (layer B.Cu) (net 6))
 (segment (start 147.5 101.3) (end 149.6 103.4) (width 0.25) (layer B.Cu) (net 6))
 (segment (start 147.5 95.5) (end 147.5 101.3) (width 0.25) (layer B.Cu) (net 6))
 (segment (start 146.165 94.165) (end 147.5 95.5) (width 0.25) (layer B.Cu) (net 6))
 (segment (start 145.075 94.165) (end 146.165 94.165) (width 0.25) (layer B.Cu) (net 6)))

